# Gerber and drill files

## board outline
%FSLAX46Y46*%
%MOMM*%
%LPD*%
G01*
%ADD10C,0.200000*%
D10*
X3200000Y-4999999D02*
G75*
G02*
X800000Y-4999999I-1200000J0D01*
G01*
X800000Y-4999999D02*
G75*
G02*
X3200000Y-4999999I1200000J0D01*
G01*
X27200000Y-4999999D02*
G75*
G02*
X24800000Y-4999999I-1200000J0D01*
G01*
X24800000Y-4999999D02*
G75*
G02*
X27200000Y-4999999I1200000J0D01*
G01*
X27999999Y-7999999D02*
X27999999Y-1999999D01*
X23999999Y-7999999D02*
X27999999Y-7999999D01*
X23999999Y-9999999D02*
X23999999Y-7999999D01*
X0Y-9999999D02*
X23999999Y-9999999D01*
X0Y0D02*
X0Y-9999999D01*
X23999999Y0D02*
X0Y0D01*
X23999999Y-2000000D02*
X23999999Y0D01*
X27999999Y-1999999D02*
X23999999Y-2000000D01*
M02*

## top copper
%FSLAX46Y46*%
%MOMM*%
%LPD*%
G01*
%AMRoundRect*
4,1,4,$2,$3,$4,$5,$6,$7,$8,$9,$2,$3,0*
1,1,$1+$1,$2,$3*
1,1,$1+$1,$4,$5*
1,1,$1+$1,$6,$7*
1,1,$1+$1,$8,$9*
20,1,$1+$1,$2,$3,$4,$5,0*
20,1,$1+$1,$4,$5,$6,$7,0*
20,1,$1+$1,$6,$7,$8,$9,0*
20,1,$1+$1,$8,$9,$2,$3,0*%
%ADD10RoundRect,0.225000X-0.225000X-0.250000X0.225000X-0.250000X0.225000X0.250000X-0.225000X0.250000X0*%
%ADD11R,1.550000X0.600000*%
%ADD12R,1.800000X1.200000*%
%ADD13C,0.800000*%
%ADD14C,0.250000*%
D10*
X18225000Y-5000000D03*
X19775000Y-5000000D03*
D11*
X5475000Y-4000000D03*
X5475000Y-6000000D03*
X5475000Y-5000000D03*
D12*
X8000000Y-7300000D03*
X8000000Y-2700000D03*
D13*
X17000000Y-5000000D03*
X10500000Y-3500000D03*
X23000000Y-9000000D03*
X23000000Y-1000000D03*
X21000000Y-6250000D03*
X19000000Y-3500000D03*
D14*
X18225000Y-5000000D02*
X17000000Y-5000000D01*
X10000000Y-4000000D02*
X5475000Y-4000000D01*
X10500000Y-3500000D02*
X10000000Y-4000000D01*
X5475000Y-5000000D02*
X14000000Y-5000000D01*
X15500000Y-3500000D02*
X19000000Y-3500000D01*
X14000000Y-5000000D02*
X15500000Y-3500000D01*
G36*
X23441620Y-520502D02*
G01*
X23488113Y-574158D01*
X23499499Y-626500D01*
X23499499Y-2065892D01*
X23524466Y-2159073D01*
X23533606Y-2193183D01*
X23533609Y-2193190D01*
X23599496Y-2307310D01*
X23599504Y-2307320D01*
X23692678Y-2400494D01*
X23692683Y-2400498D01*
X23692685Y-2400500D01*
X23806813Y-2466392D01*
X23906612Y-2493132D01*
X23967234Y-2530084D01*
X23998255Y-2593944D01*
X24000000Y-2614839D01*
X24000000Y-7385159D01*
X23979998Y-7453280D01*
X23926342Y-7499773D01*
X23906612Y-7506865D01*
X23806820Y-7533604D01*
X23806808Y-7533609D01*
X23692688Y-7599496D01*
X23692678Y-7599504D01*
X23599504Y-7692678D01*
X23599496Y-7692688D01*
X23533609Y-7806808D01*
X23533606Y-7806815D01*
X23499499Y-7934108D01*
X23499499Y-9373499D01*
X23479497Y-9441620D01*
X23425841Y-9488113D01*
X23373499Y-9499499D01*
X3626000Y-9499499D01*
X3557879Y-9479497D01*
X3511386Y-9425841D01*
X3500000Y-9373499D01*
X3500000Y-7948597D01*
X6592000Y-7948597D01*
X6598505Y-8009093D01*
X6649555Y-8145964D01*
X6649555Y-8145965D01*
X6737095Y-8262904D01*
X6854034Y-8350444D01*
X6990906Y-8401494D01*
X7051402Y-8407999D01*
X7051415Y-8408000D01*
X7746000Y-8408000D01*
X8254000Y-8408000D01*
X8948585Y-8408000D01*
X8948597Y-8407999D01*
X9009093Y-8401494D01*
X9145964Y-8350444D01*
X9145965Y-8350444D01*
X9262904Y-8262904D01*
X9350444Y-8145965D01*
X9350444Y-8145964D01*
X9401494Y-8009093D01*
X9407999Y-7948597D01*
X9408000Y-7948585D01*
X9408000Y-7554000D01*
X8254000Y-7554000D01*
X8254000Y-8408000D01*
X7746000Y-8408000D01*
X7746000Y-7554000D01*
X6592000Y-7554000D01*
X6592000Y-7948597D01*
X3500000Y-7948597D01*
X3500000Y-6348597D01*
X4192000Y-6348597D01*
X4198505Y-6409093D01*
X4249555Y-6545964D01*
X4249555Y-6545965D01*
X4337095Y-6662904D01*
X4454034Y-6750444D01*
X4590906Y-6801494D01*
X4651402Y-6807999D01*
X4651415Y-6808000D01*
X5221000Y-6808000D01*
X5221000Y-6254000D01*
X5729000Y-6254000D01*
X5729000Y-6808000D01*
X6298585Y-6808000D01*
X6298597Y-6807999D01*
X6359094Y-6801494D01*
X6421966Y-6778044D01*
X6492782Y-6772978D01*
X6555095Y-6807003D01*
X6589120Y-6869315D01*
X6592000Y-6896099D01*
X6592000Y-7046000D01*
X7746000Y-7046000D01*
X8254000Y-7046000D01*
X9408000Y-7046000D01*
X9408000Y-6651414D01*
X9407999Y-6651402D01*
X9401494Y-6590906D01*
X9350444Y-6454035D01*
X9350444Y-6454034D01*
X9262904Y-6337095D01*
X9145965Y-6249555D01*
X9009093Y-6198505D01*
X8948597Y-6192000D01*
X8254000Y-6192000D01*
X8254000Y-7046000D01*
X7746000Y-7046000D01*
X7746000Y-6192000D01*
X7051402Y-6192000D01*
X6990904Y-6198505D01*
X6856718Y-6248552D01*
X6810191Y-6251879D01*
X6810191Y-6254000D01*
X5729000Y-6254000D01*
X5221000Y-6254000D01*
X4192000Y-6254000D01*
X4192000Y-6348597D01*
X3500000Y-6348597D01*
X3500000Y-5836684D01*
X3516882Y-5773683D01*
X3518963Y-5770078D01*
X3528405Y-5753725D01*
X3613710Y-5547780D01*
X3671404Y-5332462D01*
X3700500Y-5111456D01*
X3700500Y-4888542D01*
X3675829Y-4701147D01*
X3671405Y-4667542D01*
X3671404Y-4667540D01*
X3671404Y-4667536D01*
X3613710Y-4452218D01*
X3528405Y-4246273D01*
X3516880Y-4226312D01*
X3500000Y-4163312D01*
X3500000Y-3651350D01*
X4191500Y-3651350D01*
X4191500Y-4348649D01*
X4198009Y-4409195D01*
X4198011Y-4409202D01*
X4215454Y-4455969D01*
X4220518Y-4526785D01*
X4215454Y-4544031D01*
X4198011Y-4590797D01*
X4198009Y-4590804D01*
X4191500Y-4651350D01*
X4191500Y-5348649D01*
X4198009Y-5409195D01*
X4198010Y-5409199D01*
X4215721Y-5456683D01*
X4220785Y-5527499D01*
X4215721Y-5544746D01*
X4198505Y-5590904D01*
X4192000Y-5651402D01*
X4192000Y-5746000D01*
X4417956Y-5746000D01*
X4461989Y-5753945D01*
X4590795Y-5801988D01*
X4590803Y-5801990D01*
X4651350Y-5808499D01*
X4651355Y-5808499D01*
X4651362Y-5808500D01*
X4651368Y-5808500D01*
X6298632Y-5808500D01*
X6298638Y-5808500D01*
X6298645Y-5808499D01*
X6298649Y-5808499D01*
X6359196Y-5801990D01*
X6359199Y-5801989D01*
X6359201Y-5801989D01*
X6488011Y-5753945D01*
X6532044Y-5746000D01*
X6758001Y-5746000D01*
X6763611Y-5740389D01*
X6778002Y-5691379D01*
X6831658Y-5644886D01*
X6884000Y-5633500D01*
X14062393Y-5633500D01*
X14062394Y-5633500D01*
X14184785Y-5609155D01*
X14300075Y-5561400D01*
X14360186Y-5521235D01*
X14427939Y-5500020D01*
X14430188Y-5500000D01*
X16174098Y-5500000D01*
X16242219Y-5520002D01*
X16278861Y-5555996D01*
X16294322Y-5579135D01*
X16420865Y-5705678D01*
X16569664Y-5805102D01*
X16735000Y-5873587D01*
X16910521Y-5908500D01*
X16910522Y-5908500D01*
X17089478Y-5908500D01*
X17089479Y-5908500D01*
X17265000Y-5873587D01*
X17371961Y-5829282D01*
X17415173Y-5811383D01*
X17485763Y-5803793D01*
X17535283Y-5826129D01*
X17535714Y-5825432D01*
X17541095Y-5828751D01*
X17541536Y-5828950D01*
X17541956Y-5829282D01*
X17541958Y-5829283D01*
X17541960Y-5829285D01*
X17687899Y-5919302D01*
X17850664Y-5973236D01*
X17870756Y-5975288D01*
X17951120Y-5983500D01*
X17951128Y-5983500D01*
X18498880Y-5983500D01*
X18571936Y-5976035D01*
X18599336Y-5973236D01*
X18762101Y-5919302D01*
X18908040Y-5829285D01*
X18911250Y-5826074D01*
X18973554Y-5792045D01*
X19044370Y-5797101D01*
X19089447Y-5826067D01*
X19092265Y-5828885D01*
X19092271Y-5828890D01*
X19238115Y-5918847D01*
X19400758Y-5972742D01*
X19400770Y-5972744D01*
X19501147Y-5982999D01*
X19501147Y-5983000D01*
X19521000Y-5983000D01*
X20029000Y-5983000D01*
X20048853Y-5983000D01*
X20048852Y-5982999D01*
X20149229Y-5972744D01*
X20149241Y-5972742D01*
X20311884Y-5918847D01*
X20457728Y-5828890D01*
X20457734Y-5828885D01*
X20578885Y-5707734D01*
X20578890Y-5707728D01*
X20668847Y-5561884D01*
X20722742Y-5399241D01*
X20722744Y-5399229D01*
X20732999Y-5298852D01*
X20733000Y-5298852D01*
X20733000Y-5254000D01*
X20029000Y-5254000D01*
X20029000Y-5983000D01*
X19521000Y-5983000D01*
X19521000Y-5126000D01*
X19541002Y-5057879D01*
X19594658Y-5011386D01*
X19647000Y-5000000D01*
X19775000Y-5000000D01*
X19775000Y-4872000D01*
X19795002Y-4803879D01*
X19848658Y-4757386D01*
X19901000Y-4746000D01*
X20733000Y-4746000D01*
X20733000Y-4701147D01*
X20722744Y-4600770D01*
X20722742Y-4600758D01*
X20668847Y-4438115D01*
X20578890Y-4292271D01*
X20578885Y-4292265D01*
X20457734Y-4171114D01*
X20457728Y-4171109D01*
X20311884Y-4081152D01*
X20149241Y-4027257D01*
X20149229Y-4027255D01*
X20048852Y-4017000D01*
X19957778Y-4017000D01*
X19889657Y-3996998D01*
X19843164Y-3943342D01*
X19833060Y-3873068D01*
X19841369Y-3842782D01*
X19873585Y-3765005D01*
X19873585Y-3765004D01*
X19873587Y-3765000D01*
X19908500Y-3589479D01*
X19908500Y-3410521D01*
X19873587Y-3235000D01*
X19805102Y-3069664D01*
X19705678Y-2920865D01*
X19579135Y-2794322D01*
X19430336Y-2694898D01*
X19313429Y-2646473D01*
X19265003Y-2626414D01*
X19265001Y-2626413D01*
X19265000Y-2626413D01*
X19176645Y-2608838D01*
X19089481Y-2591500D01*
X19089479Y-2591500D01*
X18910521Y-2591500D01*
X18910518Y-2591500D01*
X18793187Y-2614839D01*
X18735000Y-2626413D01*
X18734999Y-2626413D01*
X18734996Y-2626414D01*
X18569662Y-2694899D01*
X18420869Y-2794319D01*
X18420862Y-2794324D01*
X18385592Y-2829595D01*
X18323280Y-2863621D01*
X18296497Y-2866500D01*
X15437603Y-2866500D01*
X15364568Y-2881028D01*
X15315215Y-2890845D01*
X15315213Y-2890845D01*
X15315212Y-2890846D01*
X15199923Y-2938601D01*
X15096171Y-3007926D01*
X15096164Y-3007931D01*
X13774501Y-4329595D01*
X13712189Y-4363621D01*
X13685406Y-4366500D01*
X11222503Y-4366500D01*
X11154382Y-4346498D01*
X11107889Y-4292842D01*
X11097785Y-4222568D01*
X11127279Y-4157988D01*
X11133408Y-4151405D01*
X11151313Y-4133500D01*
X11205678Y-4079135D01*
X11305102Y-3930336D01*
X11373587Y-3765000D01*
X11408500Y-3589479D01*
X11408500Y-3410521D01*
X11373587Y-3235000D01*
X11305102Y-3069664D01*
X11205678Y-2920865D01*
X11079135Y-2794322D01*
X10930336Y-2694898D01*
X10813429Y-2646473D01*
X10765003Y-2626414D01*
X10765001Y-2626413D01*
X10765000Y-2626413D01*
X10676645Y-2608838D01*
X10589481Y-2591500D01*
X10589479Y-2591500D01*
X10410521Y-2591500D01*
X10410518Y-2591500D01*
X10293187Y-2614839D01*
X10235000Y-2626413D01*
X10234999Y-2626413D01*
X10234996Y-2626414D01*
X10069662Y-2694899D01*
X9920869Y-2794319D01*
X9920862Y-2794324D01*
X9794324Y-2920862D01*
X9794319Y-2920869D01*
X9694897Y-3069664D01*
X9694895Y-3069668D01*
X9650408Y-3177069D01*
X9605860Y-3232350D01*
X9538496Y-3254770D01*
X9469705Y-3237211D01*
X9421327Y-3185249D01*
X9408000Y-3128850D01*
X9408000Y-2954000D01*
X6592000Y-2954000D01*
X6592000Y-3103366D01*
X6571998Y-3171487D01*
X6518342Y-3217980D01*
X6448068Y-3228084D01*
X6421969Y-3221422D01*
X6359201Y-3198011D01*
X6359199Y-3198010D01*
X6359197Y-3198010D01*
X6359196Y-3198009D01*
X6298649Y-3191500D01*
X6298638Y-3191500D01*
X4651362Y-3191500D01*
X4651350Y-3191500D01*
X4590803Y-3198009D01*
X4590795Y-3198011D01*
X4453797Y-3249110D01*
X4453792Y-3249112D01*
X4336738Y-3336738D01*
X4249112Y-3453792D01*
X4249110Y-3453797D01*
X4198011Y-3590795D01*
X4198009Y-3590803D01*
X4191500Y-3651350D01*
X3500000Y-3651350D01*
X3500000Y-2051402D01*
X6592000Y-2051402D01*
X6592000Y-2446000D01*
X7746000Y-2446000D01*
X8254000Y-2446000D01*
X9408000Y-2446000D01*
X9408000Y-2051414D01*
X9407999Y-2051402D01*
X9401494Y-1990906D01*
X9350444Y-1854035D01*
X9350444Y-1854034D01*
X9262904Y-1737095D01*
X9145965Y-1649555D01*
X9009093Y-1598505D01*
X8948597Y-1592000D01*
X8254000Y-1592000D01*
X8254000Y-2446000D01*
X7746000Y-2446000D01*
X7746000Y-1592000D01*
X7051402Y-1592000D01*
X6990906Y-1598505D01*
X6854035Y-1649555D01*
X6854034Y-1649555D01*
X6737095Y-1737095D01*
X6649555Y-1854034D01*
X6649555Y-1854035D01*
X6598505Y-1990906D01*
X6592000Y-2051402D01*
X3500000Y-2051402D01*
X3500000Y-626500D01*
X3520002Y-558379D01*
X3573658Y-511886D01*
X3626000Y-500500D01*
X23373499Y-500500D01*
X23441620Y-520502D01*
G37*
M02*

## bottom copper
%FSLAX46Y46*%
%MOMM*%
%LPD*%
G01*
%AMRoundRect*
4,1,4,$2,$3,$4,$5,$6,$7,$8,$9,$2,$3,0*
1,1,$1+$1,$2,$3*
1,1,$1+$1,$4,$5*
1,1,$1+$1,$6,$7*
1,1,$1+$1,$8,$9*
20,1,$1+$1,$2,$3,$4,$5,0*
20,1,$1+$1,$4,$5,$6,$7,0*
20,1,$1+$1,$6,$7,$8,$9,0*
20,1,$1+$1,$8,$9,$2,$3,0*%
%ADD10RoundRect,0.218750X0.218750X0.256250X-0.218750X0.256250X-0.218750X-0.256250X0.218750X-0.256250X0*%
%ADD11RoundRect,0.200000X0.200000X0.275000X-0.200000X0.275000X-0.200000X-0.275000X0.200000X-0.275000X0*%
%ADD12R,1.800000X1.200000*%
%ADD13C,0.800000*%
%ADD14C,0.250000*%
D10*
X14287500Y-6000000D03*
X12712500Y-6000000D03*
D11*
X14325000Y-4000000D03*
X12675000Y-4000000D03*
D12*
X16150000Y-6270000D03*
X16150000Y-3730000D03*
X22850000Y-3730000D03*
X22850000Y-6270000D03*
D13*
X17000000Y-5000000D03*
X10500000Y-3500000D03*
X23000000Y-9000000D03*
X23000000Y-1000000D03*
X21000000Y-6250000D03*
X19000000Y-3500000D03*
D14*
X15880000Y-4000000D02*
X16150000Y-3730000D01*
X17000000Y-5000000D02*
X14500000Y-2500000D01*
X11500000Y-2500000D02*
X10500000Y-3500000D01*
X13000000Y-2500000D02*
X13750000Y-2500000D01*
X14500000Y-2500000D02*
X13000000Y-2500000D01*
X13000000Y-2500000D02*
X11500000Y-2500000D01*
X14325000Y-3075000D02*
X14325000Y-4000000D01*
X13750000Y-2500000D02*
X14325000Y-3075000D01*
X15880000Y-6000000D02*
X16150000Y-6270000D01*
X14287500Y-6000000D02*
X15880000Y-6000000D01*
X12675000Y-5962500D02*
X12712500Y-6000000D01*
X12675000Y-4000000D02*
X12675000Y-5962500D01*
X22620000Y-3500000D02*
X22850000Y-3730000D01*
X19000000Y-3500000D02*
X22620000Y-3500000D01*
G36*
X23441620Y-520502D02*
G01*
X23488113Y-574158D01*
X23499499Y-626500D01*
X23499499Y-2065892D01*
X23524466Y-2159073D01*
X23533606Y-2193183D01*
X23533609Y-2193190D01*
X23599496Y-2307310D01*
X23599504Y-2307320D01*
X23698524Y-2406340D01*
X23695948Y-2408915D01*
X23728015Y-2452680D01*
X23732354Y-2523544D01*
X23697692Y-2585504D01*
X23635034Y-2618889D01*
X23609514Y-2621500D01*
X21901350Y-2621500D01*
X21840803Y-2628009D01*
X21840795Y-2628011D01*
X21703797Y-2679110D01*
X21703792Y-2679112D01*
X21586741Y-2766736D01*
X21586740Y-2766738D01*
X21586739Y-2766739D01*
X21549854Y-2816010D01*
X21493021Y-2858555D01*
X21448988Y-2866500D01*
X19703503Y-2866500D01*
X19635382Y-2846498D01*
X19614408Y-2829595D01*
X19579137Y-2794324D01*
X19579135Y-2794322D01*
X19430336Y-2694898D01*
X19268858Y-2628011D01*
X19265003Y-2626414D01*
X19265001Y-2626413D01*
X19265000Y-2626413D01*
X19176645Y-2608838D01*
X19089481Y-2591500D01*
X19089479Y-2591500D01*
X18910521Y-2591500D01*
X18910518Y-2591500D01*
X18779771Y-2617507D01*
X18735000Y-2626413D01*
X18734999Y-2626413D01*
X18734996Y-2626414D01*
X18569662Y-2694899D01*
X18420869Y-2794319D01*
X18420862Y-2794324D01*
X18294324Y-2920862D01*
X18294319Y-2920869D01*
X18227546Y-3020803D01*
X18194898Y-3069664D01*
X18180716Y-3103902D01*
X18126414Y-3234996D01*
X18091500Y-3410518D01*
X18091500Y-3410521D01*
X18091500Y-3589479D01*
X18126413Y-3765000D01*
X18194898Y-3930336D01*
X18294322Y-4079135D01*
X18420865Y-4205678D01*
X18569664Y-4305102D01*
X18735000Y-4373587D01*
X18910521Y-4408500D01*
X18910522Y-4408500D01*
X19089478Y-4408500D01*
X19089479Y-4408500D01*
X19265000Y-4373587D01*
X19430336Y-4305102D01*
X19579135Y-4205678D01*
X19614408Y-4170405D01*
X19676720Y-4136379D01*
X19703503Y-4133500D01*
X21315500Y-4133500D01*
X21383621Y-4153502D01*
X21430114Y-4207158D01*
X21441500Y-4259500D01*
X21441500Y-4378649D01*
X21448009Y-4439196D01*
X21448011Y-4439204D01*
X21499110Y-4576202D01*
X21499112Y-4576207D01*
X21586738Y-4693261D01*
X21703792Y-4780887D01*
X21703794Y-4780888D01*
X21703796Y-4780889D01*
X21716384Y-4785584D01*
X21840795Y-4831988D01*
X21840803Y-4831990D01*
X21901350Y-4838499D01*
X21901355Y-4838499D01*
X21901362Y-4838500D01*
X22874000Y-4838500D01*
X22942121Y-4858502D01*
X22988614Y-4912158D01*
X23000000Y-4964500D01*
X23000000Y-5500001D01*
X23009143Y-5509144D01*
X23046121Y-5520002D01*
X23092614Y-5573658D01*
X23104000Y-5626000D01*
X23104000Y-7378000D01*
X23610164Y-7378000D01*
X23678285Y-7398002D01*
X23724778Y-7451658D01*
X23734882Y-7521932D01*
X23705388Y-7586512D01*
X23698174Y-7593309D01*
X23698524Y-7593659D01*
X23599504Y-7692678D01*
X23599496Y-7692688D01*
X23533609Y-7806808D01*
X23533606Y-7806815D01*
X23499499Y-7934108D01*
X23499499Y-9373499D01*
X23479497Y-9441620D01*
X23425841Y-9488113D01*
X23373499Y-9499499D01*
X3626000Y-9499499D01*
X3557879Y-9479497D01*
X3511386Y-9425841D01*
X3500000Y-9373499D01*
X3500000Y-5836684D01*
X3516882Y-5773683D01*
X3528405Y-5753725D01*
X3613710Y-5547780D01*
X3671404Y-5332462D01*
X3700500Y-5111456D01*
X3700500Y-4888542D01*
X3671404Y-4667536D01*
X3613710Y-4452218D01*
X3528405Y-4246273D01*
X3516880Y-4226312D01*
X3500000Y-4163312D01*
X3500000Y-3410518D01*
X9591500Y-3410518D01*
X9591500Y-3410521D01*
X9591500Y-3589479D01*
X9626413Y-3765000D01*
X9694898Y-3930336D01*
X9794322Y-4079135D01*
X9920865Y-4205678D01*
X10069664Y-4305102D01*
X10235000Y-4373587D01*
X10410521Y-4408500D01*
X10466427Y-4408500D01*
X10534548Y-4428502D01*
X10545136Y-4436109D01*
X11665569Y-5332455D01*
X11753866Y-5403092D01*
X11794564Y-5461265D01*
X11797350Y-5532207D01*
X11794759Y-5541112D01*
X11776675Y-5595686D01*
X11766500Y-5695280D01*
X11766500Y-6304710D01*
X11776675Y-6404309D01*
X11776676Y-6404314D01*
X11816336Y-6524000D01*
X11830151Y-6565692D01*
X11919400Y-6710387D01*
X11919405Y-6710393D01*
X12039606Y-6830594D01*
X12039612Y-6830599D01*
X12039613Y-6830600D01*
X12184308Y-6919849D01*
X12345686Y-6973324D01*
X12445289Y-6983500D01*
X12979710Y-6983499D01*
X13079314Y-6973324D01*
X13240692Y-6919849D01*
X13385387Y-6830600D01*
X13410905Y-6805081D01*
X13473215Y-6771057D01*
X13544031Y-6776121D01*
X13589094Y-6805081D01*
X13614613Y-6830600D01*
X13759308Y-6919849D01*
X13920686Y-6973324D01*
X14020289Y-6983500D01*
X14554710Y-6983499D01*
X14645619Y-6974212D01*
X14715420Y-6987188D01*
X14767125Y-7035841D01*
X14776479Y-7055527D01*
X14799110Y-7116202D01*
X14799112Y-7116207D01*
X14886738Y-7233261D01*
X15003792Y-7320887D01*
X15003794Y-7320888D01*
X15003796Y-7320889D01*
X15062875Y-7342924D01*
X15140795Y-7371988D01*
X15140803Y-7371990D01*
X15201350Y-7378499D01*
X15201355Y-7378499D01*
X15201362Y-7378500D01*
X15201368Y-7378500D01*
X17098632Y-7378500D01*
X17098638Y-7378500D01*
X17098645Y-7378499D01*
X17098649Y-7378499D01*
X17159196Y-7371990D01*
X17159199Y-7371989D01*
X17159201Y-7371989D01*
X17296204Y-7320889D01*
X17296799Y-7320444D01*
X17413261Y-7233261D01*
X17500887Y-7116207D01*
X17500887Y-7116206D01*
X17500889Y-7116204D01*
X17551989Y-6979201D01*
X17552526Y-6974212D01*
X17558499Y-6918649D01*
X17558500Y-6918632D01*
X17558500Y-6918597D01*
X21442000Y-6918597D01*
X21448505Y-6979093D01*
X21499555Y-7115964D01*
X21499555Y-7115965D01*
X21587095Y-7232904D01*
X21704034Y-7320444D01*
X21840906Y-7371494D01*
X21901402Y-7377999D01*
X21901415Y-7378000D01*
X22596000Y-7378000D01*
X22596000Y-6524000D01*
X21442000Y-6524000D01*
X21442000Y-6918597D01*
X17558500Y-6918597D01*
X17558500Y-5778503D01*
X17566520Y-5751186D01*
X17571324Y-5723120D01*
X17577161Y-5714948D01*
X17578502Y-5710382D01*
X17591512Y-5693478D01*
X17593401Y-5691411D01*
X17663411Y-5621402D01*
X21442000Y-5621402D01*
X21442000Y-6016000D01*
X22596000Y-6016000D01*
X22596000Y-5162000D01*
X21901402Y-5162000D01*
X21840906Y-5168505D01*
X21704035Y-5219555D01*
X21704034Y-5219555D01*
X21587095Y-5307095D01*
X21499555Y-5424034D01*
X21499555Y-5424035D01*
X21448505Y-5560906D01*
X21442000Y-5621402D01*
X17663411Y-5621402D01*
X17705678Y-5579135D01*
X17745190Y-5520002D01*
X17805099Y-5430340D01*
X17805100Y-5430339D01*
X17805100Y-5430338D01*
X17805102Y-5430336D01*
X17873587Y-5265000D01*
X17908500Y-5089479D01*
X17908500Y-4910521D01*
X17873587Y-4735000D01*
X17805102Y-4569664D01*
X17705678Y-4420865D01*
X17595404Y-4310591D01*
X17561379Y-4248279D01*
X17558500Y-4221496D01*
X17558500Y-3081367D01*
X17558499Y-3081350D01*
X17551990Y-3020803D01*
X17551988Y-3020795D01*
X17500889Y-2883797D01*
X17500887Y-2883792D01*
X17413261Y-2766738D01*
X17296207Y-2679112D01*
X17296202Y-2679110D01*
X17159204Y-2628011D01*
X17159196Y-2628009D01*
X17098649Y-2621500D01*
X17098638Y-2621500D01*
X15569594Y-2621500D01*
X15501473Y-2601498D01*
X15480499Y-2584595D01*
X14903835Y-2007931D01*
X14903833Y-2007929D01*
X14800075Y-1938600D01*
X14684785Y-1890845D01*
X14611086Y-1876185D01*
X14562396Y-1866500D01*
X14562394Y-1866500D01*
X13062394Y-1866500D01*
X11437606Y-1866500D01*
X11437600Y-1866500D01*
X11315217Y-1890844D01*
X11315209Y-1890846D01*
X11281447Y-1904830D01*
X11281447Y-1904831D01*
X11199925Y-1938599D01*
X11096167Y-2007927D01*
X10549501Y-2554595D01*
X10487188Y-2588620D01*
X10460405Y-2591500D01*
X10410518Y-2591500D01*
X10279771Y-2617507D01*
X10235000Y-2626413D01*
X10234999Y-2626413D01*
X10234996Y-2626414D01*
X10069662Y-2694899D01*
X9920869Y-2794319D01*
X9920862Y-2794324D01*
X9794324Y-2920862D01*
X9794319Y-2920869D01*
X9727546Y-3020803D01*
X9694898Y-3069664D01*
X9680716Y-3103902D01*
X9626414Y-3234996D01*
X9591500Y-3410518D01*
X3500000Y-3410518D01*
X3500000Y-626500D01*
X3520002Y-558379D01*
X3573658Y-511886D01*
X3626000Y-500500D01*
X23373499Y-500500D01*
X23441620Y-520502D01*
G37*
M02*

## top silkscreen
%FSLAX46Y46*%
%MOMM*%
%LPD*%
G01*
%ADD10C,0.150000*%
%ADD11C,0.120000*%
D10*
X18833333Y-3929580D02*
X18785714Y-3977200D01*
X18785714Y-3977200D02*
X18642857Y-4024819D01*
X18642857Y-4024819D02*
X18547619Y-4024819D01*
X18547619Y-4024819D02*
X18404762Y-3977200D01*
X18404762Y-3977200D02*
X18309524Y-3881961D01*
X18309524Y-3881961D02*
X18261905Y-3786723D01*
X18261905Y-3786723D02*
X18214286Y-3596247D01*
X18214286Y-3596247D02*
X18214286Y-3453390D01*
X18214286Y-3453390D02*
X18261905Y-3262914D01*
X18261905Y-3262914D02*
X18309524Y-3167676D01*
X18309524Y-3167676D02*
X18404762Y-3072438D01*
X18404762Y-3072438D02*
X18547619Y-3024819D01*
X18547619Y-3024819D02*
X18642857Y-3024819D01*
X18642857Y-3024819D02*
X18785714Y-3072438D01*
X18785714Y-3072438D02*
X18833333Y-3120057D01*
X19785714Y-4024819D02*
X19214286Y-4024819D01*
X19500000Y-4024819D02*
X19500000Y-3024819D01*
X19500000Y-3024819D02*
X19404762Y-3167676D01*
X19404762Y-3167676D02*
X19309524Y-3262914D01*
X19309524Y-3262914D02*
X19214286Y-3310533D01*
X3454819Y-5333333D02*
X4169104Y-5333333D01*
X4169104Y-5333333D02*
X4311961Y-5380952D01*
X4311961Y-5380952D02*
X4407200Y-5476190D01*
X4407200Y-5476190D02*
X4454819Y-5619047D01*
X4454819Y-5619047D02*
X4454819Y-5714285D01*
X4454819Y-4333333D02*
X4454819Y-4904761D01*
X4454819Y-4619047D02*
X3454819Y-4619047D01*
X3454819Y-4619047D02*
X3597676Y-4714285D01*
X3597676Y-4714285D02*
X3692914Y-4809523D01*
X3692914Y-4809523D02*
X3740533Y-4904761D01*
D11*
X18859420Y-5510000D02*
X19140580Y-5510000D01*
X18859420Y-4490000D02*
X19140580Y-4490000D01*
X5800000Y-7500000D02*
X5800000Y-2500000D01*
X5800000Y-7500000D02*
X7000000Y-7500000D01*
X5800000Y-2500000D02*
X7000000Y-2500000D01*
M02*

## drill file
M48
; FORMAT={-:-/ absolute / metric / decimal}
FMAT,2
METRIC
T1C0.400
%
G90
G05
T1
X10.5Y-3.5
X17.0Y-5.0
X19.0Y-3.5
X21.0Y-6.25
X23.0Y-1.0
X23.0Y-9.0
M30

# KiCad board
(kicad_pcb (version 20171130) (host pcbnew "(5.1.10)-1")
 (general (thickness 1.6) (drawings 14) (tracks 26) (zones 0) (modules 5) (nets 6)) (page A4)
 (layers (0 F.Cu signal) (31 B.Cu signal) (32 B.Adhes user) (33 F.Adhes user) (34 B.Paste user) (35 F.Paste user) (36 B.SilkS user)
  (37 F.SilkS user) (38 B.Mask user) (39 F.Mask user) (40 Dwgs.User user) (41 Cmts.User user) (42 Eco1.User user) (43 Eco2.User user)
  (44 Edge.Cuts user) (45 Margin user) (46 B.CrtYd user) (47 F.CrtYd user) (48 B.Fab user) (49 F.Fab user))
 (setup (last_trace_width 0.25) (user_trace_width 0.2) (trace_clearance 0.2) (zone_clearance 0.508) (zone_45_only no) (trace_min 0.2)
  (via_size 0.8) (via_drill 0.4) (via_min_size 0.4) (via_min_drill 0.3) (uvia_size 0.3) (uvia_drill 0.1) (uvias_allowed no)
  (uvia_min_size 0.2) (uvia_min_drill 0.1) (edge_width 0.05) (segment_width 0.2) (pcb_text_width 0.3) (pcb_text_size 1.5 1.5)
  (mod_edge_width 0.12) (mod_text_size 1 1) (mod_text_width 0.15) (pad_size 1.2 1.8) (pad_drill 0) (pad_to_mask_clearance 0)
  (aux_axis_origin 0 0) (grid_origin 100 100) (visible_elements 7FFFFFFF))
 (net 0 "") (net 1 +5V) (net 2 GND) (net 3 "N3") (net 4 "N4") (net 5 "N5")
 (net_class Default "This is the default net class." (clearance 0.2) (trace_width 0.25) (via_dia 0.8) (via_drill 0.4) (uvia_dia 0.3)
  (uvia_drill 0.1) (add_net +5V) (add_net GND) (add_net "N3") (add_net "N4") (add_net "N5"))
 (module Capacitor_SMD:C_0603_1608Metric (layer F.Cu) (at 19 5)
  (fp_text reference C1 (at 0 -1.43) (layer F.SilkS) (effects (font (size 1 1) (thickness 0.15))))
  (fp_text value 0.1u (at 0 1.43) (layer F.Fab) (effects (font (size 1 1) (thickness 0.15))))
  (fp_line (start -0.14058 0.51) (end 0.14058 0.51) (layer F.SilkS) (width 0.12))
  (fp_line (start -0.14058 -0.51) (end 0.14058 -0.51) (layer F.SilkS) (width 0.12))
  (pad 1 smd roundrect (at -0.775 0) (size 0.9 0.95) (layers F.Cu F.Paste F.Mask) (roundrect_rratio 0.25) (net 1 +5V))
  (pad 2 smd roundrect (at 0.775 0) (size 0.9 0.95) (layers F.Cu F.Paste F.Mask) (roundrect_rratio 0.25) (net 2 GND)))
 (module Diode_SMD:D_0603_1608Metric (layer B.Cu) (at 13.5 6 180)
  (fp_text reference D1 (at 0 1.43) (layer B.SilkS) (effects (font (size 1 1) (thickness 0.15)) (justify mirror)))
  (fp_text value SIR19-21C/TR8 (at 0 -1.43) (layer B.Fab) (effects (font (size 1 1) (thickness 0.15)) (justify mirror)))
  (pad 1 smd roundrect (at -0.7875 0 180) (size 0.875 0.95) (layers B.Cu B.Paste B.Mask) (roundrect_rratio 0.25) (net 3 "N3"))
  (pad 2 smd roundrect (at 0.7875 0 180) (size 0.875 0.95) (layers B.Cu B.Paste B.Mask) (roundrect_rratio 0.25) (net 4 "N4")))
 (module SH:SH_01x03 (layer F.Cu) (at 8 5 90)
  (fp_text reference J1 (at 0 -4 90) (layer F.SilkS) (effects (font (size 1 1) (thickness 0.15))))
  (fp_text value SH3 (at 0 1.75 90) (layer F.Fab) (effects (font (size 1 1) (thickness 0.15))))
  (fp_line (start -2.5 -2.2) (end 2.5 -2.2) (layer F.SilkS) (width 0.12))
  (fp_line (start -2.5 -2.2) (end -2.5 -1) (layer F.SilkS) (width 0.12))
  (fp_line (start 2.5 -2.2) (end 2.5 -1) (layer F.SilkS) (width 0.12))
  (pad 3 smd rect (at 1 -2.525 90) (size 0.6 1.55) (layers F.Cu F.Paste F.Mask) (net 1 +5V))
  (pad 1 smd rect (at -1 -2.525 90) (size 0.6 1.55) (layers F.Cu F.Paste F.Mask) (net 2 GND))
  (pad 2 smd rect (at 0 -2.525 90) (size 0.6 1.55) (layers F.Cu F.Paste F.Mask) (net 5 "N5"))
  (pad MP smd rect (at -2.3 0 90) (size 1.2 1.8) (layers F.Cu F.Paste F.Mask) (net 2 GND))
  (pad MP smd rect (at 2.3 0 90) (size 1.2 1.8) (layers F.Cu F.Paste F.Mask) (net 2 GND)))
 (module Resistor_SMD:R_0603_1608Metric (layer B.Cu) (at 13.5 4 180)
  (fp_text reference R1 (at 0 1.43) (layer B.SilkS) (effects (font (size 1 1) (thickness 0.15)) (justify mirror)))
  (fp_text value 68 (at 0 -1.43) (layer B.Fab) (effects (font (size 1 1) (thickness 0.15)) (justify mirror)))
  (pad 1 smd roundrect (at -0.825 0 180) (size 0.8 0.95) (layers B.Cu B.Paste B.Mask) (roundrect_rratio 0.25) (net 1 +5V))
  (pad 2 smd roundrect (at 0.825 0 180) (size 0.8 0.95) (layers B.Cu B.Paste B.Mask) (roundrect_rratio 0.25) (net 4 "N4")))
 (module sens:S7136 (layer B.Cu) (at 19.5 5)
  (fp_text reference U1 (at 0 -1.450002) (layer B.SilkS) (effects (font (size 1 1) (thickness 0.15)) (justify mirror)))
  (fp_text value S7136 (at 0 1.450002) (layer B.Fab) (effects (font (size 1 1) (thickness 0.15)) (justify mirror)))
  (pad 1 smd rect (at -3.35 1.27) (size 1.8 1.2) (layers B.Cu B.Paste B.Mask) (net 3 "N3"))
  (pad 2 smd rect (at -3.35 -1.27) (size 1.8 1.2) (layers B.Cu B.Paste B.Mask) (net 1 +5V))
  (pad 3 smd rect (at 3.35 -1.27) (size 1.8 1.2) (layers B.Cu B.Paste B.Mask) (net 5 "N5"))
  (pad 4 smd rect (at 3.35 1.27) (size 1.8 1.2) (layers B.Cu B.Paste B.Mask) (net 2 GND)))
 (gr_circle (center 2 4.999999) (end 3.2 4.999999) (layer Edge.Cuts) (width 0.2))
 (gr_circle (center 26 4.999999) (end 27.2 4.999999) (layer Edge.Cuts) (width 0.2))
 (gr_line (start 27.999999 7.999999) (end 27.999999 1.999999) (layer Edge.Cuts) (width 0.2))
 (gr_line (start 23.999999 7.999999) (end 27.999999 7.999999) (layer Edge.Cuts) (width 0.2))
 (gr_line (start 23.999999 9.999999) (end 23.999999 7.999999) (layer Edge.Cuts) (width 0.2))
 (gr_line (start 0 9.999999) (end 23.999999 9.999999) (layer Edge.Cuts) (width 0.2))
 (gr_line (start 0 0) (end 0 9.999999) (layer Edge.Cuts) (width 0.2))
 (gr_line (start 23.999999 0) (end 0 0) (layer Edge.Cuts) (width 0.2))
 (gr_line (start 23.999999 2) (end 23.999999 0) (layer Edge.Cuts) (width 0.2))
 (gr_line (start 27.999999 1.999999) (end 23.999999 2) (layer Edge.Cuts) (width 0.2))
 (segment (start 15.88 4) (end 16.15 3.73) (width 0.25) (layer B.Cu) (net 1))
 (via (at 17 5) (size 0.8) (drill 0.4) (layers F.Cu B.Cu) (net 1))
 (segment (start 18.225 5) (end 17 5) (width 0.25) (layer F.Cu) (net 1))
 (segment (start 17 5) (end 14.5 2.5) (width 0.25) (layer B.Cu) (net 1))
 (via (at 10.5 3.5) (size 0.8) (drill 0.4) (layers F.Cu B.Cu) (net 1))
 (segment (start 11.5 2.5) (end 10.5 3.5) (width 0.25) (layer B.Cu) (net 1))
 (segment (start 10 4) (end 5.475 4) (width 0.25) (layer F.Cu) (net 1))
 (segment (start 10.5 3.5) (end 10 4) (width 0.25) (layer F.Cu) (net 1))
 (segment (start 13 2.5) (end 13.75 2.5) (width 0.25) (layer B.Cu) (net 1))
 (segment (start 14.5 2.5) (end 13 2.5) (width 0.25) (layer B.Cu) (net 1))
 (segment (start 13 2.5) (end 11.5 2.5) (width 0.25) (layer B.Cu) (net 1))
 (segment (start 14.325 3.075) (end 14.325 4) (width 0.25) (layer B.Cu) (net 1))
 (segment (start 13.75 2.5) (end 14.325 3.075) (width 0.25) (layer B.Cu) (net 1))
 (via (at 23 9) (size 0.8) (drill 0.4) (layers F.Cu B.Cu) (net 2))
 (via (at 23 1) (size 0.8) (drill 0.4) (layers F.Cu B.Cu) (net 2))
 (via (at 21 6.25) (size 0.8) (drill 0.4) (layers F.Cu B.Cu) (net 2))
 (segment (start 15.88 6) (end 16.15 6.27) (width 0.25) (layer B.Cu) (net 3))
 (segment (start 14.2875 6) (end 15.88 6) (width 0.25) (layer B.Cu) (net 3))
 (segment (start 12.675 5.9625) (end 12.7125 6) (width 0.25) (layer B.Cu) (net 4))
 (segment (start 12.675 4) (end 12.675 5.9625) (width 0.25) (layer B.Cu) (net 4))
 (segment (start 5.475 5) (end 14 5) (width 0.25) (layer F.Cu) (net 5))
 (via (at 19 3.5) (size 0.8) (drill 0.4) (layers F.Cu B.Cu) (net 5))
 (segment (start 15.5 3.5) (end 19 3.5) (width 0.25) (layer F.Cu) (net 5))
 (segment (start 14 5) (end 15.5 3.5) (width 0.25) (layer F.Cu) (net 5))
 (segment (start 22.62 3.5) (end 22.85 3.73) (width 0.25) (layer B.Cu) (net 5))
 (segment (start 19 3.5) (end 22.62 3.5) (width 0.25) (layer B.Cu) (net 5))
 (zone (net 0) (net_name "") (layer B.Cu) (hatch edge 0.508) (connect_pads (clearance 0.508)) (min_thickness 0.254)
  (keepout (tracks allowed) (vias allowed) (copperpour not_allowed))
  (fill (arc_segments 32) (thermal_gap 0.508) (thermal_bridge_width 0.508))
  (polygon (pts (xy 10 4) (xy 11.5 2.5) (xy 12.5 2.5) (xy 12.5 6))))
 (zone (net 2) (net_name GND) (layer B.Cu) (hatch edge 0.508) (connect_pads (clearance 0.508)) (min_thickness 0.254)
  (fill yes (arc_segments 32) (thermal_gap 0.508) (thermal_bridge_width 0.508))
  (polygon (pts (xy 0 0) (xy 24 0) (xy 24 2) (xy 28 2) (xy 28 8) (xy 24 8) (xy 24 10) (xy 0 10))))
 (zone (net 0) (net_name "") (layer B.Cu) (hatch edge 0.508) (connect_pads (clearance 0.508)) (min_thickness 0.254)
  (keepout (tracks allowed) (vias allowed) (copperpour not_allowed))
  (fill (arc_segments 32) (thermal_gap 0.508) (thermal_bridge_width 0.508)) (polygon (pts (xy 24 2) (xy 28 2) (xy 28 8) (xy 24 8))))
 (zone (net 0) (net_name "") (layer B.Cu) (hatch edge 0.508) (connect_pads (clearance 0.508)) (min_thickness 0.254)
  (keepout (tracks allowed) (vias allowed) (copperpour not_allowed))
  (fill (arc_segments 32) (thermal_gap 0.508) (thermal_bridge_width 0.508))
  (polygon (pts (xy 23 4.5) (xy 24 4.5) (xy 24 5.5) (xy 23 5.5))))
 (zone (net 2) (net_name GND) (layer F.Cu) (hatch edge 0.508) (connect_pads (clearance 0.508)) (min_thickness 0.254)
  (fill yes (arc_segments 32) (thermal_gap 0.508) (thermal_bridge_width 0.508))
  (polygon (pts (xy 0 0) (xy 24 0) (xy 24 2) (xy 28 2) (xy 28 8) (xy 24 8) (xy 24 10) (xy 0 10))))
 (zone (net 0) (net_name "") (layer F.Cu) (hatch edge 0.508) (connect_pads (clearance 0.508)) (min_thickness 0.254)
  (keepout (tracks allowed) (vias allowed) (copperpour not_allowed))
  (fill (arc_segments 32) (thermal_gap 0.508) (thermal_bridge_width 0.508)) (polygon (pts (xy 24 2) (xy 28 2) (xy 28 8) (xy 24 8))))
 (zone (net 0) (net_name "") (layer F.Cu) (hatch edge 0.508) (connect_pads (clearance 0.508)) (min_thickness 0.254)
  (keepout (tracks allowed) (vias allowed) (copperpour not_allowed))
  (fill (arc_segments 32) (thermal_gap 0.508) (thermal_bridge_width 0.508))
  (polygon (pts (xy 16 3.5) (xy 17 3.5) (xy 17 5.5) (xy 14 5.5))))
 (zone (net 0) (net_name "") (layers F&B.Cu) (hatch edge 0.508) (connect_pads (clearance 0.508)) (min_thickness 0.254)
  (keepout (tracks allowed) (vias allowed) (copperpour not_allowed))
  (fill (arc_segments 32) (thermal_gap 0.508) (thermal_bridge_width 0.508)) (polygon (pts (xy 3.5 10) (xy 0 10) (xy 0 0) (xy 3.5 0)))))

